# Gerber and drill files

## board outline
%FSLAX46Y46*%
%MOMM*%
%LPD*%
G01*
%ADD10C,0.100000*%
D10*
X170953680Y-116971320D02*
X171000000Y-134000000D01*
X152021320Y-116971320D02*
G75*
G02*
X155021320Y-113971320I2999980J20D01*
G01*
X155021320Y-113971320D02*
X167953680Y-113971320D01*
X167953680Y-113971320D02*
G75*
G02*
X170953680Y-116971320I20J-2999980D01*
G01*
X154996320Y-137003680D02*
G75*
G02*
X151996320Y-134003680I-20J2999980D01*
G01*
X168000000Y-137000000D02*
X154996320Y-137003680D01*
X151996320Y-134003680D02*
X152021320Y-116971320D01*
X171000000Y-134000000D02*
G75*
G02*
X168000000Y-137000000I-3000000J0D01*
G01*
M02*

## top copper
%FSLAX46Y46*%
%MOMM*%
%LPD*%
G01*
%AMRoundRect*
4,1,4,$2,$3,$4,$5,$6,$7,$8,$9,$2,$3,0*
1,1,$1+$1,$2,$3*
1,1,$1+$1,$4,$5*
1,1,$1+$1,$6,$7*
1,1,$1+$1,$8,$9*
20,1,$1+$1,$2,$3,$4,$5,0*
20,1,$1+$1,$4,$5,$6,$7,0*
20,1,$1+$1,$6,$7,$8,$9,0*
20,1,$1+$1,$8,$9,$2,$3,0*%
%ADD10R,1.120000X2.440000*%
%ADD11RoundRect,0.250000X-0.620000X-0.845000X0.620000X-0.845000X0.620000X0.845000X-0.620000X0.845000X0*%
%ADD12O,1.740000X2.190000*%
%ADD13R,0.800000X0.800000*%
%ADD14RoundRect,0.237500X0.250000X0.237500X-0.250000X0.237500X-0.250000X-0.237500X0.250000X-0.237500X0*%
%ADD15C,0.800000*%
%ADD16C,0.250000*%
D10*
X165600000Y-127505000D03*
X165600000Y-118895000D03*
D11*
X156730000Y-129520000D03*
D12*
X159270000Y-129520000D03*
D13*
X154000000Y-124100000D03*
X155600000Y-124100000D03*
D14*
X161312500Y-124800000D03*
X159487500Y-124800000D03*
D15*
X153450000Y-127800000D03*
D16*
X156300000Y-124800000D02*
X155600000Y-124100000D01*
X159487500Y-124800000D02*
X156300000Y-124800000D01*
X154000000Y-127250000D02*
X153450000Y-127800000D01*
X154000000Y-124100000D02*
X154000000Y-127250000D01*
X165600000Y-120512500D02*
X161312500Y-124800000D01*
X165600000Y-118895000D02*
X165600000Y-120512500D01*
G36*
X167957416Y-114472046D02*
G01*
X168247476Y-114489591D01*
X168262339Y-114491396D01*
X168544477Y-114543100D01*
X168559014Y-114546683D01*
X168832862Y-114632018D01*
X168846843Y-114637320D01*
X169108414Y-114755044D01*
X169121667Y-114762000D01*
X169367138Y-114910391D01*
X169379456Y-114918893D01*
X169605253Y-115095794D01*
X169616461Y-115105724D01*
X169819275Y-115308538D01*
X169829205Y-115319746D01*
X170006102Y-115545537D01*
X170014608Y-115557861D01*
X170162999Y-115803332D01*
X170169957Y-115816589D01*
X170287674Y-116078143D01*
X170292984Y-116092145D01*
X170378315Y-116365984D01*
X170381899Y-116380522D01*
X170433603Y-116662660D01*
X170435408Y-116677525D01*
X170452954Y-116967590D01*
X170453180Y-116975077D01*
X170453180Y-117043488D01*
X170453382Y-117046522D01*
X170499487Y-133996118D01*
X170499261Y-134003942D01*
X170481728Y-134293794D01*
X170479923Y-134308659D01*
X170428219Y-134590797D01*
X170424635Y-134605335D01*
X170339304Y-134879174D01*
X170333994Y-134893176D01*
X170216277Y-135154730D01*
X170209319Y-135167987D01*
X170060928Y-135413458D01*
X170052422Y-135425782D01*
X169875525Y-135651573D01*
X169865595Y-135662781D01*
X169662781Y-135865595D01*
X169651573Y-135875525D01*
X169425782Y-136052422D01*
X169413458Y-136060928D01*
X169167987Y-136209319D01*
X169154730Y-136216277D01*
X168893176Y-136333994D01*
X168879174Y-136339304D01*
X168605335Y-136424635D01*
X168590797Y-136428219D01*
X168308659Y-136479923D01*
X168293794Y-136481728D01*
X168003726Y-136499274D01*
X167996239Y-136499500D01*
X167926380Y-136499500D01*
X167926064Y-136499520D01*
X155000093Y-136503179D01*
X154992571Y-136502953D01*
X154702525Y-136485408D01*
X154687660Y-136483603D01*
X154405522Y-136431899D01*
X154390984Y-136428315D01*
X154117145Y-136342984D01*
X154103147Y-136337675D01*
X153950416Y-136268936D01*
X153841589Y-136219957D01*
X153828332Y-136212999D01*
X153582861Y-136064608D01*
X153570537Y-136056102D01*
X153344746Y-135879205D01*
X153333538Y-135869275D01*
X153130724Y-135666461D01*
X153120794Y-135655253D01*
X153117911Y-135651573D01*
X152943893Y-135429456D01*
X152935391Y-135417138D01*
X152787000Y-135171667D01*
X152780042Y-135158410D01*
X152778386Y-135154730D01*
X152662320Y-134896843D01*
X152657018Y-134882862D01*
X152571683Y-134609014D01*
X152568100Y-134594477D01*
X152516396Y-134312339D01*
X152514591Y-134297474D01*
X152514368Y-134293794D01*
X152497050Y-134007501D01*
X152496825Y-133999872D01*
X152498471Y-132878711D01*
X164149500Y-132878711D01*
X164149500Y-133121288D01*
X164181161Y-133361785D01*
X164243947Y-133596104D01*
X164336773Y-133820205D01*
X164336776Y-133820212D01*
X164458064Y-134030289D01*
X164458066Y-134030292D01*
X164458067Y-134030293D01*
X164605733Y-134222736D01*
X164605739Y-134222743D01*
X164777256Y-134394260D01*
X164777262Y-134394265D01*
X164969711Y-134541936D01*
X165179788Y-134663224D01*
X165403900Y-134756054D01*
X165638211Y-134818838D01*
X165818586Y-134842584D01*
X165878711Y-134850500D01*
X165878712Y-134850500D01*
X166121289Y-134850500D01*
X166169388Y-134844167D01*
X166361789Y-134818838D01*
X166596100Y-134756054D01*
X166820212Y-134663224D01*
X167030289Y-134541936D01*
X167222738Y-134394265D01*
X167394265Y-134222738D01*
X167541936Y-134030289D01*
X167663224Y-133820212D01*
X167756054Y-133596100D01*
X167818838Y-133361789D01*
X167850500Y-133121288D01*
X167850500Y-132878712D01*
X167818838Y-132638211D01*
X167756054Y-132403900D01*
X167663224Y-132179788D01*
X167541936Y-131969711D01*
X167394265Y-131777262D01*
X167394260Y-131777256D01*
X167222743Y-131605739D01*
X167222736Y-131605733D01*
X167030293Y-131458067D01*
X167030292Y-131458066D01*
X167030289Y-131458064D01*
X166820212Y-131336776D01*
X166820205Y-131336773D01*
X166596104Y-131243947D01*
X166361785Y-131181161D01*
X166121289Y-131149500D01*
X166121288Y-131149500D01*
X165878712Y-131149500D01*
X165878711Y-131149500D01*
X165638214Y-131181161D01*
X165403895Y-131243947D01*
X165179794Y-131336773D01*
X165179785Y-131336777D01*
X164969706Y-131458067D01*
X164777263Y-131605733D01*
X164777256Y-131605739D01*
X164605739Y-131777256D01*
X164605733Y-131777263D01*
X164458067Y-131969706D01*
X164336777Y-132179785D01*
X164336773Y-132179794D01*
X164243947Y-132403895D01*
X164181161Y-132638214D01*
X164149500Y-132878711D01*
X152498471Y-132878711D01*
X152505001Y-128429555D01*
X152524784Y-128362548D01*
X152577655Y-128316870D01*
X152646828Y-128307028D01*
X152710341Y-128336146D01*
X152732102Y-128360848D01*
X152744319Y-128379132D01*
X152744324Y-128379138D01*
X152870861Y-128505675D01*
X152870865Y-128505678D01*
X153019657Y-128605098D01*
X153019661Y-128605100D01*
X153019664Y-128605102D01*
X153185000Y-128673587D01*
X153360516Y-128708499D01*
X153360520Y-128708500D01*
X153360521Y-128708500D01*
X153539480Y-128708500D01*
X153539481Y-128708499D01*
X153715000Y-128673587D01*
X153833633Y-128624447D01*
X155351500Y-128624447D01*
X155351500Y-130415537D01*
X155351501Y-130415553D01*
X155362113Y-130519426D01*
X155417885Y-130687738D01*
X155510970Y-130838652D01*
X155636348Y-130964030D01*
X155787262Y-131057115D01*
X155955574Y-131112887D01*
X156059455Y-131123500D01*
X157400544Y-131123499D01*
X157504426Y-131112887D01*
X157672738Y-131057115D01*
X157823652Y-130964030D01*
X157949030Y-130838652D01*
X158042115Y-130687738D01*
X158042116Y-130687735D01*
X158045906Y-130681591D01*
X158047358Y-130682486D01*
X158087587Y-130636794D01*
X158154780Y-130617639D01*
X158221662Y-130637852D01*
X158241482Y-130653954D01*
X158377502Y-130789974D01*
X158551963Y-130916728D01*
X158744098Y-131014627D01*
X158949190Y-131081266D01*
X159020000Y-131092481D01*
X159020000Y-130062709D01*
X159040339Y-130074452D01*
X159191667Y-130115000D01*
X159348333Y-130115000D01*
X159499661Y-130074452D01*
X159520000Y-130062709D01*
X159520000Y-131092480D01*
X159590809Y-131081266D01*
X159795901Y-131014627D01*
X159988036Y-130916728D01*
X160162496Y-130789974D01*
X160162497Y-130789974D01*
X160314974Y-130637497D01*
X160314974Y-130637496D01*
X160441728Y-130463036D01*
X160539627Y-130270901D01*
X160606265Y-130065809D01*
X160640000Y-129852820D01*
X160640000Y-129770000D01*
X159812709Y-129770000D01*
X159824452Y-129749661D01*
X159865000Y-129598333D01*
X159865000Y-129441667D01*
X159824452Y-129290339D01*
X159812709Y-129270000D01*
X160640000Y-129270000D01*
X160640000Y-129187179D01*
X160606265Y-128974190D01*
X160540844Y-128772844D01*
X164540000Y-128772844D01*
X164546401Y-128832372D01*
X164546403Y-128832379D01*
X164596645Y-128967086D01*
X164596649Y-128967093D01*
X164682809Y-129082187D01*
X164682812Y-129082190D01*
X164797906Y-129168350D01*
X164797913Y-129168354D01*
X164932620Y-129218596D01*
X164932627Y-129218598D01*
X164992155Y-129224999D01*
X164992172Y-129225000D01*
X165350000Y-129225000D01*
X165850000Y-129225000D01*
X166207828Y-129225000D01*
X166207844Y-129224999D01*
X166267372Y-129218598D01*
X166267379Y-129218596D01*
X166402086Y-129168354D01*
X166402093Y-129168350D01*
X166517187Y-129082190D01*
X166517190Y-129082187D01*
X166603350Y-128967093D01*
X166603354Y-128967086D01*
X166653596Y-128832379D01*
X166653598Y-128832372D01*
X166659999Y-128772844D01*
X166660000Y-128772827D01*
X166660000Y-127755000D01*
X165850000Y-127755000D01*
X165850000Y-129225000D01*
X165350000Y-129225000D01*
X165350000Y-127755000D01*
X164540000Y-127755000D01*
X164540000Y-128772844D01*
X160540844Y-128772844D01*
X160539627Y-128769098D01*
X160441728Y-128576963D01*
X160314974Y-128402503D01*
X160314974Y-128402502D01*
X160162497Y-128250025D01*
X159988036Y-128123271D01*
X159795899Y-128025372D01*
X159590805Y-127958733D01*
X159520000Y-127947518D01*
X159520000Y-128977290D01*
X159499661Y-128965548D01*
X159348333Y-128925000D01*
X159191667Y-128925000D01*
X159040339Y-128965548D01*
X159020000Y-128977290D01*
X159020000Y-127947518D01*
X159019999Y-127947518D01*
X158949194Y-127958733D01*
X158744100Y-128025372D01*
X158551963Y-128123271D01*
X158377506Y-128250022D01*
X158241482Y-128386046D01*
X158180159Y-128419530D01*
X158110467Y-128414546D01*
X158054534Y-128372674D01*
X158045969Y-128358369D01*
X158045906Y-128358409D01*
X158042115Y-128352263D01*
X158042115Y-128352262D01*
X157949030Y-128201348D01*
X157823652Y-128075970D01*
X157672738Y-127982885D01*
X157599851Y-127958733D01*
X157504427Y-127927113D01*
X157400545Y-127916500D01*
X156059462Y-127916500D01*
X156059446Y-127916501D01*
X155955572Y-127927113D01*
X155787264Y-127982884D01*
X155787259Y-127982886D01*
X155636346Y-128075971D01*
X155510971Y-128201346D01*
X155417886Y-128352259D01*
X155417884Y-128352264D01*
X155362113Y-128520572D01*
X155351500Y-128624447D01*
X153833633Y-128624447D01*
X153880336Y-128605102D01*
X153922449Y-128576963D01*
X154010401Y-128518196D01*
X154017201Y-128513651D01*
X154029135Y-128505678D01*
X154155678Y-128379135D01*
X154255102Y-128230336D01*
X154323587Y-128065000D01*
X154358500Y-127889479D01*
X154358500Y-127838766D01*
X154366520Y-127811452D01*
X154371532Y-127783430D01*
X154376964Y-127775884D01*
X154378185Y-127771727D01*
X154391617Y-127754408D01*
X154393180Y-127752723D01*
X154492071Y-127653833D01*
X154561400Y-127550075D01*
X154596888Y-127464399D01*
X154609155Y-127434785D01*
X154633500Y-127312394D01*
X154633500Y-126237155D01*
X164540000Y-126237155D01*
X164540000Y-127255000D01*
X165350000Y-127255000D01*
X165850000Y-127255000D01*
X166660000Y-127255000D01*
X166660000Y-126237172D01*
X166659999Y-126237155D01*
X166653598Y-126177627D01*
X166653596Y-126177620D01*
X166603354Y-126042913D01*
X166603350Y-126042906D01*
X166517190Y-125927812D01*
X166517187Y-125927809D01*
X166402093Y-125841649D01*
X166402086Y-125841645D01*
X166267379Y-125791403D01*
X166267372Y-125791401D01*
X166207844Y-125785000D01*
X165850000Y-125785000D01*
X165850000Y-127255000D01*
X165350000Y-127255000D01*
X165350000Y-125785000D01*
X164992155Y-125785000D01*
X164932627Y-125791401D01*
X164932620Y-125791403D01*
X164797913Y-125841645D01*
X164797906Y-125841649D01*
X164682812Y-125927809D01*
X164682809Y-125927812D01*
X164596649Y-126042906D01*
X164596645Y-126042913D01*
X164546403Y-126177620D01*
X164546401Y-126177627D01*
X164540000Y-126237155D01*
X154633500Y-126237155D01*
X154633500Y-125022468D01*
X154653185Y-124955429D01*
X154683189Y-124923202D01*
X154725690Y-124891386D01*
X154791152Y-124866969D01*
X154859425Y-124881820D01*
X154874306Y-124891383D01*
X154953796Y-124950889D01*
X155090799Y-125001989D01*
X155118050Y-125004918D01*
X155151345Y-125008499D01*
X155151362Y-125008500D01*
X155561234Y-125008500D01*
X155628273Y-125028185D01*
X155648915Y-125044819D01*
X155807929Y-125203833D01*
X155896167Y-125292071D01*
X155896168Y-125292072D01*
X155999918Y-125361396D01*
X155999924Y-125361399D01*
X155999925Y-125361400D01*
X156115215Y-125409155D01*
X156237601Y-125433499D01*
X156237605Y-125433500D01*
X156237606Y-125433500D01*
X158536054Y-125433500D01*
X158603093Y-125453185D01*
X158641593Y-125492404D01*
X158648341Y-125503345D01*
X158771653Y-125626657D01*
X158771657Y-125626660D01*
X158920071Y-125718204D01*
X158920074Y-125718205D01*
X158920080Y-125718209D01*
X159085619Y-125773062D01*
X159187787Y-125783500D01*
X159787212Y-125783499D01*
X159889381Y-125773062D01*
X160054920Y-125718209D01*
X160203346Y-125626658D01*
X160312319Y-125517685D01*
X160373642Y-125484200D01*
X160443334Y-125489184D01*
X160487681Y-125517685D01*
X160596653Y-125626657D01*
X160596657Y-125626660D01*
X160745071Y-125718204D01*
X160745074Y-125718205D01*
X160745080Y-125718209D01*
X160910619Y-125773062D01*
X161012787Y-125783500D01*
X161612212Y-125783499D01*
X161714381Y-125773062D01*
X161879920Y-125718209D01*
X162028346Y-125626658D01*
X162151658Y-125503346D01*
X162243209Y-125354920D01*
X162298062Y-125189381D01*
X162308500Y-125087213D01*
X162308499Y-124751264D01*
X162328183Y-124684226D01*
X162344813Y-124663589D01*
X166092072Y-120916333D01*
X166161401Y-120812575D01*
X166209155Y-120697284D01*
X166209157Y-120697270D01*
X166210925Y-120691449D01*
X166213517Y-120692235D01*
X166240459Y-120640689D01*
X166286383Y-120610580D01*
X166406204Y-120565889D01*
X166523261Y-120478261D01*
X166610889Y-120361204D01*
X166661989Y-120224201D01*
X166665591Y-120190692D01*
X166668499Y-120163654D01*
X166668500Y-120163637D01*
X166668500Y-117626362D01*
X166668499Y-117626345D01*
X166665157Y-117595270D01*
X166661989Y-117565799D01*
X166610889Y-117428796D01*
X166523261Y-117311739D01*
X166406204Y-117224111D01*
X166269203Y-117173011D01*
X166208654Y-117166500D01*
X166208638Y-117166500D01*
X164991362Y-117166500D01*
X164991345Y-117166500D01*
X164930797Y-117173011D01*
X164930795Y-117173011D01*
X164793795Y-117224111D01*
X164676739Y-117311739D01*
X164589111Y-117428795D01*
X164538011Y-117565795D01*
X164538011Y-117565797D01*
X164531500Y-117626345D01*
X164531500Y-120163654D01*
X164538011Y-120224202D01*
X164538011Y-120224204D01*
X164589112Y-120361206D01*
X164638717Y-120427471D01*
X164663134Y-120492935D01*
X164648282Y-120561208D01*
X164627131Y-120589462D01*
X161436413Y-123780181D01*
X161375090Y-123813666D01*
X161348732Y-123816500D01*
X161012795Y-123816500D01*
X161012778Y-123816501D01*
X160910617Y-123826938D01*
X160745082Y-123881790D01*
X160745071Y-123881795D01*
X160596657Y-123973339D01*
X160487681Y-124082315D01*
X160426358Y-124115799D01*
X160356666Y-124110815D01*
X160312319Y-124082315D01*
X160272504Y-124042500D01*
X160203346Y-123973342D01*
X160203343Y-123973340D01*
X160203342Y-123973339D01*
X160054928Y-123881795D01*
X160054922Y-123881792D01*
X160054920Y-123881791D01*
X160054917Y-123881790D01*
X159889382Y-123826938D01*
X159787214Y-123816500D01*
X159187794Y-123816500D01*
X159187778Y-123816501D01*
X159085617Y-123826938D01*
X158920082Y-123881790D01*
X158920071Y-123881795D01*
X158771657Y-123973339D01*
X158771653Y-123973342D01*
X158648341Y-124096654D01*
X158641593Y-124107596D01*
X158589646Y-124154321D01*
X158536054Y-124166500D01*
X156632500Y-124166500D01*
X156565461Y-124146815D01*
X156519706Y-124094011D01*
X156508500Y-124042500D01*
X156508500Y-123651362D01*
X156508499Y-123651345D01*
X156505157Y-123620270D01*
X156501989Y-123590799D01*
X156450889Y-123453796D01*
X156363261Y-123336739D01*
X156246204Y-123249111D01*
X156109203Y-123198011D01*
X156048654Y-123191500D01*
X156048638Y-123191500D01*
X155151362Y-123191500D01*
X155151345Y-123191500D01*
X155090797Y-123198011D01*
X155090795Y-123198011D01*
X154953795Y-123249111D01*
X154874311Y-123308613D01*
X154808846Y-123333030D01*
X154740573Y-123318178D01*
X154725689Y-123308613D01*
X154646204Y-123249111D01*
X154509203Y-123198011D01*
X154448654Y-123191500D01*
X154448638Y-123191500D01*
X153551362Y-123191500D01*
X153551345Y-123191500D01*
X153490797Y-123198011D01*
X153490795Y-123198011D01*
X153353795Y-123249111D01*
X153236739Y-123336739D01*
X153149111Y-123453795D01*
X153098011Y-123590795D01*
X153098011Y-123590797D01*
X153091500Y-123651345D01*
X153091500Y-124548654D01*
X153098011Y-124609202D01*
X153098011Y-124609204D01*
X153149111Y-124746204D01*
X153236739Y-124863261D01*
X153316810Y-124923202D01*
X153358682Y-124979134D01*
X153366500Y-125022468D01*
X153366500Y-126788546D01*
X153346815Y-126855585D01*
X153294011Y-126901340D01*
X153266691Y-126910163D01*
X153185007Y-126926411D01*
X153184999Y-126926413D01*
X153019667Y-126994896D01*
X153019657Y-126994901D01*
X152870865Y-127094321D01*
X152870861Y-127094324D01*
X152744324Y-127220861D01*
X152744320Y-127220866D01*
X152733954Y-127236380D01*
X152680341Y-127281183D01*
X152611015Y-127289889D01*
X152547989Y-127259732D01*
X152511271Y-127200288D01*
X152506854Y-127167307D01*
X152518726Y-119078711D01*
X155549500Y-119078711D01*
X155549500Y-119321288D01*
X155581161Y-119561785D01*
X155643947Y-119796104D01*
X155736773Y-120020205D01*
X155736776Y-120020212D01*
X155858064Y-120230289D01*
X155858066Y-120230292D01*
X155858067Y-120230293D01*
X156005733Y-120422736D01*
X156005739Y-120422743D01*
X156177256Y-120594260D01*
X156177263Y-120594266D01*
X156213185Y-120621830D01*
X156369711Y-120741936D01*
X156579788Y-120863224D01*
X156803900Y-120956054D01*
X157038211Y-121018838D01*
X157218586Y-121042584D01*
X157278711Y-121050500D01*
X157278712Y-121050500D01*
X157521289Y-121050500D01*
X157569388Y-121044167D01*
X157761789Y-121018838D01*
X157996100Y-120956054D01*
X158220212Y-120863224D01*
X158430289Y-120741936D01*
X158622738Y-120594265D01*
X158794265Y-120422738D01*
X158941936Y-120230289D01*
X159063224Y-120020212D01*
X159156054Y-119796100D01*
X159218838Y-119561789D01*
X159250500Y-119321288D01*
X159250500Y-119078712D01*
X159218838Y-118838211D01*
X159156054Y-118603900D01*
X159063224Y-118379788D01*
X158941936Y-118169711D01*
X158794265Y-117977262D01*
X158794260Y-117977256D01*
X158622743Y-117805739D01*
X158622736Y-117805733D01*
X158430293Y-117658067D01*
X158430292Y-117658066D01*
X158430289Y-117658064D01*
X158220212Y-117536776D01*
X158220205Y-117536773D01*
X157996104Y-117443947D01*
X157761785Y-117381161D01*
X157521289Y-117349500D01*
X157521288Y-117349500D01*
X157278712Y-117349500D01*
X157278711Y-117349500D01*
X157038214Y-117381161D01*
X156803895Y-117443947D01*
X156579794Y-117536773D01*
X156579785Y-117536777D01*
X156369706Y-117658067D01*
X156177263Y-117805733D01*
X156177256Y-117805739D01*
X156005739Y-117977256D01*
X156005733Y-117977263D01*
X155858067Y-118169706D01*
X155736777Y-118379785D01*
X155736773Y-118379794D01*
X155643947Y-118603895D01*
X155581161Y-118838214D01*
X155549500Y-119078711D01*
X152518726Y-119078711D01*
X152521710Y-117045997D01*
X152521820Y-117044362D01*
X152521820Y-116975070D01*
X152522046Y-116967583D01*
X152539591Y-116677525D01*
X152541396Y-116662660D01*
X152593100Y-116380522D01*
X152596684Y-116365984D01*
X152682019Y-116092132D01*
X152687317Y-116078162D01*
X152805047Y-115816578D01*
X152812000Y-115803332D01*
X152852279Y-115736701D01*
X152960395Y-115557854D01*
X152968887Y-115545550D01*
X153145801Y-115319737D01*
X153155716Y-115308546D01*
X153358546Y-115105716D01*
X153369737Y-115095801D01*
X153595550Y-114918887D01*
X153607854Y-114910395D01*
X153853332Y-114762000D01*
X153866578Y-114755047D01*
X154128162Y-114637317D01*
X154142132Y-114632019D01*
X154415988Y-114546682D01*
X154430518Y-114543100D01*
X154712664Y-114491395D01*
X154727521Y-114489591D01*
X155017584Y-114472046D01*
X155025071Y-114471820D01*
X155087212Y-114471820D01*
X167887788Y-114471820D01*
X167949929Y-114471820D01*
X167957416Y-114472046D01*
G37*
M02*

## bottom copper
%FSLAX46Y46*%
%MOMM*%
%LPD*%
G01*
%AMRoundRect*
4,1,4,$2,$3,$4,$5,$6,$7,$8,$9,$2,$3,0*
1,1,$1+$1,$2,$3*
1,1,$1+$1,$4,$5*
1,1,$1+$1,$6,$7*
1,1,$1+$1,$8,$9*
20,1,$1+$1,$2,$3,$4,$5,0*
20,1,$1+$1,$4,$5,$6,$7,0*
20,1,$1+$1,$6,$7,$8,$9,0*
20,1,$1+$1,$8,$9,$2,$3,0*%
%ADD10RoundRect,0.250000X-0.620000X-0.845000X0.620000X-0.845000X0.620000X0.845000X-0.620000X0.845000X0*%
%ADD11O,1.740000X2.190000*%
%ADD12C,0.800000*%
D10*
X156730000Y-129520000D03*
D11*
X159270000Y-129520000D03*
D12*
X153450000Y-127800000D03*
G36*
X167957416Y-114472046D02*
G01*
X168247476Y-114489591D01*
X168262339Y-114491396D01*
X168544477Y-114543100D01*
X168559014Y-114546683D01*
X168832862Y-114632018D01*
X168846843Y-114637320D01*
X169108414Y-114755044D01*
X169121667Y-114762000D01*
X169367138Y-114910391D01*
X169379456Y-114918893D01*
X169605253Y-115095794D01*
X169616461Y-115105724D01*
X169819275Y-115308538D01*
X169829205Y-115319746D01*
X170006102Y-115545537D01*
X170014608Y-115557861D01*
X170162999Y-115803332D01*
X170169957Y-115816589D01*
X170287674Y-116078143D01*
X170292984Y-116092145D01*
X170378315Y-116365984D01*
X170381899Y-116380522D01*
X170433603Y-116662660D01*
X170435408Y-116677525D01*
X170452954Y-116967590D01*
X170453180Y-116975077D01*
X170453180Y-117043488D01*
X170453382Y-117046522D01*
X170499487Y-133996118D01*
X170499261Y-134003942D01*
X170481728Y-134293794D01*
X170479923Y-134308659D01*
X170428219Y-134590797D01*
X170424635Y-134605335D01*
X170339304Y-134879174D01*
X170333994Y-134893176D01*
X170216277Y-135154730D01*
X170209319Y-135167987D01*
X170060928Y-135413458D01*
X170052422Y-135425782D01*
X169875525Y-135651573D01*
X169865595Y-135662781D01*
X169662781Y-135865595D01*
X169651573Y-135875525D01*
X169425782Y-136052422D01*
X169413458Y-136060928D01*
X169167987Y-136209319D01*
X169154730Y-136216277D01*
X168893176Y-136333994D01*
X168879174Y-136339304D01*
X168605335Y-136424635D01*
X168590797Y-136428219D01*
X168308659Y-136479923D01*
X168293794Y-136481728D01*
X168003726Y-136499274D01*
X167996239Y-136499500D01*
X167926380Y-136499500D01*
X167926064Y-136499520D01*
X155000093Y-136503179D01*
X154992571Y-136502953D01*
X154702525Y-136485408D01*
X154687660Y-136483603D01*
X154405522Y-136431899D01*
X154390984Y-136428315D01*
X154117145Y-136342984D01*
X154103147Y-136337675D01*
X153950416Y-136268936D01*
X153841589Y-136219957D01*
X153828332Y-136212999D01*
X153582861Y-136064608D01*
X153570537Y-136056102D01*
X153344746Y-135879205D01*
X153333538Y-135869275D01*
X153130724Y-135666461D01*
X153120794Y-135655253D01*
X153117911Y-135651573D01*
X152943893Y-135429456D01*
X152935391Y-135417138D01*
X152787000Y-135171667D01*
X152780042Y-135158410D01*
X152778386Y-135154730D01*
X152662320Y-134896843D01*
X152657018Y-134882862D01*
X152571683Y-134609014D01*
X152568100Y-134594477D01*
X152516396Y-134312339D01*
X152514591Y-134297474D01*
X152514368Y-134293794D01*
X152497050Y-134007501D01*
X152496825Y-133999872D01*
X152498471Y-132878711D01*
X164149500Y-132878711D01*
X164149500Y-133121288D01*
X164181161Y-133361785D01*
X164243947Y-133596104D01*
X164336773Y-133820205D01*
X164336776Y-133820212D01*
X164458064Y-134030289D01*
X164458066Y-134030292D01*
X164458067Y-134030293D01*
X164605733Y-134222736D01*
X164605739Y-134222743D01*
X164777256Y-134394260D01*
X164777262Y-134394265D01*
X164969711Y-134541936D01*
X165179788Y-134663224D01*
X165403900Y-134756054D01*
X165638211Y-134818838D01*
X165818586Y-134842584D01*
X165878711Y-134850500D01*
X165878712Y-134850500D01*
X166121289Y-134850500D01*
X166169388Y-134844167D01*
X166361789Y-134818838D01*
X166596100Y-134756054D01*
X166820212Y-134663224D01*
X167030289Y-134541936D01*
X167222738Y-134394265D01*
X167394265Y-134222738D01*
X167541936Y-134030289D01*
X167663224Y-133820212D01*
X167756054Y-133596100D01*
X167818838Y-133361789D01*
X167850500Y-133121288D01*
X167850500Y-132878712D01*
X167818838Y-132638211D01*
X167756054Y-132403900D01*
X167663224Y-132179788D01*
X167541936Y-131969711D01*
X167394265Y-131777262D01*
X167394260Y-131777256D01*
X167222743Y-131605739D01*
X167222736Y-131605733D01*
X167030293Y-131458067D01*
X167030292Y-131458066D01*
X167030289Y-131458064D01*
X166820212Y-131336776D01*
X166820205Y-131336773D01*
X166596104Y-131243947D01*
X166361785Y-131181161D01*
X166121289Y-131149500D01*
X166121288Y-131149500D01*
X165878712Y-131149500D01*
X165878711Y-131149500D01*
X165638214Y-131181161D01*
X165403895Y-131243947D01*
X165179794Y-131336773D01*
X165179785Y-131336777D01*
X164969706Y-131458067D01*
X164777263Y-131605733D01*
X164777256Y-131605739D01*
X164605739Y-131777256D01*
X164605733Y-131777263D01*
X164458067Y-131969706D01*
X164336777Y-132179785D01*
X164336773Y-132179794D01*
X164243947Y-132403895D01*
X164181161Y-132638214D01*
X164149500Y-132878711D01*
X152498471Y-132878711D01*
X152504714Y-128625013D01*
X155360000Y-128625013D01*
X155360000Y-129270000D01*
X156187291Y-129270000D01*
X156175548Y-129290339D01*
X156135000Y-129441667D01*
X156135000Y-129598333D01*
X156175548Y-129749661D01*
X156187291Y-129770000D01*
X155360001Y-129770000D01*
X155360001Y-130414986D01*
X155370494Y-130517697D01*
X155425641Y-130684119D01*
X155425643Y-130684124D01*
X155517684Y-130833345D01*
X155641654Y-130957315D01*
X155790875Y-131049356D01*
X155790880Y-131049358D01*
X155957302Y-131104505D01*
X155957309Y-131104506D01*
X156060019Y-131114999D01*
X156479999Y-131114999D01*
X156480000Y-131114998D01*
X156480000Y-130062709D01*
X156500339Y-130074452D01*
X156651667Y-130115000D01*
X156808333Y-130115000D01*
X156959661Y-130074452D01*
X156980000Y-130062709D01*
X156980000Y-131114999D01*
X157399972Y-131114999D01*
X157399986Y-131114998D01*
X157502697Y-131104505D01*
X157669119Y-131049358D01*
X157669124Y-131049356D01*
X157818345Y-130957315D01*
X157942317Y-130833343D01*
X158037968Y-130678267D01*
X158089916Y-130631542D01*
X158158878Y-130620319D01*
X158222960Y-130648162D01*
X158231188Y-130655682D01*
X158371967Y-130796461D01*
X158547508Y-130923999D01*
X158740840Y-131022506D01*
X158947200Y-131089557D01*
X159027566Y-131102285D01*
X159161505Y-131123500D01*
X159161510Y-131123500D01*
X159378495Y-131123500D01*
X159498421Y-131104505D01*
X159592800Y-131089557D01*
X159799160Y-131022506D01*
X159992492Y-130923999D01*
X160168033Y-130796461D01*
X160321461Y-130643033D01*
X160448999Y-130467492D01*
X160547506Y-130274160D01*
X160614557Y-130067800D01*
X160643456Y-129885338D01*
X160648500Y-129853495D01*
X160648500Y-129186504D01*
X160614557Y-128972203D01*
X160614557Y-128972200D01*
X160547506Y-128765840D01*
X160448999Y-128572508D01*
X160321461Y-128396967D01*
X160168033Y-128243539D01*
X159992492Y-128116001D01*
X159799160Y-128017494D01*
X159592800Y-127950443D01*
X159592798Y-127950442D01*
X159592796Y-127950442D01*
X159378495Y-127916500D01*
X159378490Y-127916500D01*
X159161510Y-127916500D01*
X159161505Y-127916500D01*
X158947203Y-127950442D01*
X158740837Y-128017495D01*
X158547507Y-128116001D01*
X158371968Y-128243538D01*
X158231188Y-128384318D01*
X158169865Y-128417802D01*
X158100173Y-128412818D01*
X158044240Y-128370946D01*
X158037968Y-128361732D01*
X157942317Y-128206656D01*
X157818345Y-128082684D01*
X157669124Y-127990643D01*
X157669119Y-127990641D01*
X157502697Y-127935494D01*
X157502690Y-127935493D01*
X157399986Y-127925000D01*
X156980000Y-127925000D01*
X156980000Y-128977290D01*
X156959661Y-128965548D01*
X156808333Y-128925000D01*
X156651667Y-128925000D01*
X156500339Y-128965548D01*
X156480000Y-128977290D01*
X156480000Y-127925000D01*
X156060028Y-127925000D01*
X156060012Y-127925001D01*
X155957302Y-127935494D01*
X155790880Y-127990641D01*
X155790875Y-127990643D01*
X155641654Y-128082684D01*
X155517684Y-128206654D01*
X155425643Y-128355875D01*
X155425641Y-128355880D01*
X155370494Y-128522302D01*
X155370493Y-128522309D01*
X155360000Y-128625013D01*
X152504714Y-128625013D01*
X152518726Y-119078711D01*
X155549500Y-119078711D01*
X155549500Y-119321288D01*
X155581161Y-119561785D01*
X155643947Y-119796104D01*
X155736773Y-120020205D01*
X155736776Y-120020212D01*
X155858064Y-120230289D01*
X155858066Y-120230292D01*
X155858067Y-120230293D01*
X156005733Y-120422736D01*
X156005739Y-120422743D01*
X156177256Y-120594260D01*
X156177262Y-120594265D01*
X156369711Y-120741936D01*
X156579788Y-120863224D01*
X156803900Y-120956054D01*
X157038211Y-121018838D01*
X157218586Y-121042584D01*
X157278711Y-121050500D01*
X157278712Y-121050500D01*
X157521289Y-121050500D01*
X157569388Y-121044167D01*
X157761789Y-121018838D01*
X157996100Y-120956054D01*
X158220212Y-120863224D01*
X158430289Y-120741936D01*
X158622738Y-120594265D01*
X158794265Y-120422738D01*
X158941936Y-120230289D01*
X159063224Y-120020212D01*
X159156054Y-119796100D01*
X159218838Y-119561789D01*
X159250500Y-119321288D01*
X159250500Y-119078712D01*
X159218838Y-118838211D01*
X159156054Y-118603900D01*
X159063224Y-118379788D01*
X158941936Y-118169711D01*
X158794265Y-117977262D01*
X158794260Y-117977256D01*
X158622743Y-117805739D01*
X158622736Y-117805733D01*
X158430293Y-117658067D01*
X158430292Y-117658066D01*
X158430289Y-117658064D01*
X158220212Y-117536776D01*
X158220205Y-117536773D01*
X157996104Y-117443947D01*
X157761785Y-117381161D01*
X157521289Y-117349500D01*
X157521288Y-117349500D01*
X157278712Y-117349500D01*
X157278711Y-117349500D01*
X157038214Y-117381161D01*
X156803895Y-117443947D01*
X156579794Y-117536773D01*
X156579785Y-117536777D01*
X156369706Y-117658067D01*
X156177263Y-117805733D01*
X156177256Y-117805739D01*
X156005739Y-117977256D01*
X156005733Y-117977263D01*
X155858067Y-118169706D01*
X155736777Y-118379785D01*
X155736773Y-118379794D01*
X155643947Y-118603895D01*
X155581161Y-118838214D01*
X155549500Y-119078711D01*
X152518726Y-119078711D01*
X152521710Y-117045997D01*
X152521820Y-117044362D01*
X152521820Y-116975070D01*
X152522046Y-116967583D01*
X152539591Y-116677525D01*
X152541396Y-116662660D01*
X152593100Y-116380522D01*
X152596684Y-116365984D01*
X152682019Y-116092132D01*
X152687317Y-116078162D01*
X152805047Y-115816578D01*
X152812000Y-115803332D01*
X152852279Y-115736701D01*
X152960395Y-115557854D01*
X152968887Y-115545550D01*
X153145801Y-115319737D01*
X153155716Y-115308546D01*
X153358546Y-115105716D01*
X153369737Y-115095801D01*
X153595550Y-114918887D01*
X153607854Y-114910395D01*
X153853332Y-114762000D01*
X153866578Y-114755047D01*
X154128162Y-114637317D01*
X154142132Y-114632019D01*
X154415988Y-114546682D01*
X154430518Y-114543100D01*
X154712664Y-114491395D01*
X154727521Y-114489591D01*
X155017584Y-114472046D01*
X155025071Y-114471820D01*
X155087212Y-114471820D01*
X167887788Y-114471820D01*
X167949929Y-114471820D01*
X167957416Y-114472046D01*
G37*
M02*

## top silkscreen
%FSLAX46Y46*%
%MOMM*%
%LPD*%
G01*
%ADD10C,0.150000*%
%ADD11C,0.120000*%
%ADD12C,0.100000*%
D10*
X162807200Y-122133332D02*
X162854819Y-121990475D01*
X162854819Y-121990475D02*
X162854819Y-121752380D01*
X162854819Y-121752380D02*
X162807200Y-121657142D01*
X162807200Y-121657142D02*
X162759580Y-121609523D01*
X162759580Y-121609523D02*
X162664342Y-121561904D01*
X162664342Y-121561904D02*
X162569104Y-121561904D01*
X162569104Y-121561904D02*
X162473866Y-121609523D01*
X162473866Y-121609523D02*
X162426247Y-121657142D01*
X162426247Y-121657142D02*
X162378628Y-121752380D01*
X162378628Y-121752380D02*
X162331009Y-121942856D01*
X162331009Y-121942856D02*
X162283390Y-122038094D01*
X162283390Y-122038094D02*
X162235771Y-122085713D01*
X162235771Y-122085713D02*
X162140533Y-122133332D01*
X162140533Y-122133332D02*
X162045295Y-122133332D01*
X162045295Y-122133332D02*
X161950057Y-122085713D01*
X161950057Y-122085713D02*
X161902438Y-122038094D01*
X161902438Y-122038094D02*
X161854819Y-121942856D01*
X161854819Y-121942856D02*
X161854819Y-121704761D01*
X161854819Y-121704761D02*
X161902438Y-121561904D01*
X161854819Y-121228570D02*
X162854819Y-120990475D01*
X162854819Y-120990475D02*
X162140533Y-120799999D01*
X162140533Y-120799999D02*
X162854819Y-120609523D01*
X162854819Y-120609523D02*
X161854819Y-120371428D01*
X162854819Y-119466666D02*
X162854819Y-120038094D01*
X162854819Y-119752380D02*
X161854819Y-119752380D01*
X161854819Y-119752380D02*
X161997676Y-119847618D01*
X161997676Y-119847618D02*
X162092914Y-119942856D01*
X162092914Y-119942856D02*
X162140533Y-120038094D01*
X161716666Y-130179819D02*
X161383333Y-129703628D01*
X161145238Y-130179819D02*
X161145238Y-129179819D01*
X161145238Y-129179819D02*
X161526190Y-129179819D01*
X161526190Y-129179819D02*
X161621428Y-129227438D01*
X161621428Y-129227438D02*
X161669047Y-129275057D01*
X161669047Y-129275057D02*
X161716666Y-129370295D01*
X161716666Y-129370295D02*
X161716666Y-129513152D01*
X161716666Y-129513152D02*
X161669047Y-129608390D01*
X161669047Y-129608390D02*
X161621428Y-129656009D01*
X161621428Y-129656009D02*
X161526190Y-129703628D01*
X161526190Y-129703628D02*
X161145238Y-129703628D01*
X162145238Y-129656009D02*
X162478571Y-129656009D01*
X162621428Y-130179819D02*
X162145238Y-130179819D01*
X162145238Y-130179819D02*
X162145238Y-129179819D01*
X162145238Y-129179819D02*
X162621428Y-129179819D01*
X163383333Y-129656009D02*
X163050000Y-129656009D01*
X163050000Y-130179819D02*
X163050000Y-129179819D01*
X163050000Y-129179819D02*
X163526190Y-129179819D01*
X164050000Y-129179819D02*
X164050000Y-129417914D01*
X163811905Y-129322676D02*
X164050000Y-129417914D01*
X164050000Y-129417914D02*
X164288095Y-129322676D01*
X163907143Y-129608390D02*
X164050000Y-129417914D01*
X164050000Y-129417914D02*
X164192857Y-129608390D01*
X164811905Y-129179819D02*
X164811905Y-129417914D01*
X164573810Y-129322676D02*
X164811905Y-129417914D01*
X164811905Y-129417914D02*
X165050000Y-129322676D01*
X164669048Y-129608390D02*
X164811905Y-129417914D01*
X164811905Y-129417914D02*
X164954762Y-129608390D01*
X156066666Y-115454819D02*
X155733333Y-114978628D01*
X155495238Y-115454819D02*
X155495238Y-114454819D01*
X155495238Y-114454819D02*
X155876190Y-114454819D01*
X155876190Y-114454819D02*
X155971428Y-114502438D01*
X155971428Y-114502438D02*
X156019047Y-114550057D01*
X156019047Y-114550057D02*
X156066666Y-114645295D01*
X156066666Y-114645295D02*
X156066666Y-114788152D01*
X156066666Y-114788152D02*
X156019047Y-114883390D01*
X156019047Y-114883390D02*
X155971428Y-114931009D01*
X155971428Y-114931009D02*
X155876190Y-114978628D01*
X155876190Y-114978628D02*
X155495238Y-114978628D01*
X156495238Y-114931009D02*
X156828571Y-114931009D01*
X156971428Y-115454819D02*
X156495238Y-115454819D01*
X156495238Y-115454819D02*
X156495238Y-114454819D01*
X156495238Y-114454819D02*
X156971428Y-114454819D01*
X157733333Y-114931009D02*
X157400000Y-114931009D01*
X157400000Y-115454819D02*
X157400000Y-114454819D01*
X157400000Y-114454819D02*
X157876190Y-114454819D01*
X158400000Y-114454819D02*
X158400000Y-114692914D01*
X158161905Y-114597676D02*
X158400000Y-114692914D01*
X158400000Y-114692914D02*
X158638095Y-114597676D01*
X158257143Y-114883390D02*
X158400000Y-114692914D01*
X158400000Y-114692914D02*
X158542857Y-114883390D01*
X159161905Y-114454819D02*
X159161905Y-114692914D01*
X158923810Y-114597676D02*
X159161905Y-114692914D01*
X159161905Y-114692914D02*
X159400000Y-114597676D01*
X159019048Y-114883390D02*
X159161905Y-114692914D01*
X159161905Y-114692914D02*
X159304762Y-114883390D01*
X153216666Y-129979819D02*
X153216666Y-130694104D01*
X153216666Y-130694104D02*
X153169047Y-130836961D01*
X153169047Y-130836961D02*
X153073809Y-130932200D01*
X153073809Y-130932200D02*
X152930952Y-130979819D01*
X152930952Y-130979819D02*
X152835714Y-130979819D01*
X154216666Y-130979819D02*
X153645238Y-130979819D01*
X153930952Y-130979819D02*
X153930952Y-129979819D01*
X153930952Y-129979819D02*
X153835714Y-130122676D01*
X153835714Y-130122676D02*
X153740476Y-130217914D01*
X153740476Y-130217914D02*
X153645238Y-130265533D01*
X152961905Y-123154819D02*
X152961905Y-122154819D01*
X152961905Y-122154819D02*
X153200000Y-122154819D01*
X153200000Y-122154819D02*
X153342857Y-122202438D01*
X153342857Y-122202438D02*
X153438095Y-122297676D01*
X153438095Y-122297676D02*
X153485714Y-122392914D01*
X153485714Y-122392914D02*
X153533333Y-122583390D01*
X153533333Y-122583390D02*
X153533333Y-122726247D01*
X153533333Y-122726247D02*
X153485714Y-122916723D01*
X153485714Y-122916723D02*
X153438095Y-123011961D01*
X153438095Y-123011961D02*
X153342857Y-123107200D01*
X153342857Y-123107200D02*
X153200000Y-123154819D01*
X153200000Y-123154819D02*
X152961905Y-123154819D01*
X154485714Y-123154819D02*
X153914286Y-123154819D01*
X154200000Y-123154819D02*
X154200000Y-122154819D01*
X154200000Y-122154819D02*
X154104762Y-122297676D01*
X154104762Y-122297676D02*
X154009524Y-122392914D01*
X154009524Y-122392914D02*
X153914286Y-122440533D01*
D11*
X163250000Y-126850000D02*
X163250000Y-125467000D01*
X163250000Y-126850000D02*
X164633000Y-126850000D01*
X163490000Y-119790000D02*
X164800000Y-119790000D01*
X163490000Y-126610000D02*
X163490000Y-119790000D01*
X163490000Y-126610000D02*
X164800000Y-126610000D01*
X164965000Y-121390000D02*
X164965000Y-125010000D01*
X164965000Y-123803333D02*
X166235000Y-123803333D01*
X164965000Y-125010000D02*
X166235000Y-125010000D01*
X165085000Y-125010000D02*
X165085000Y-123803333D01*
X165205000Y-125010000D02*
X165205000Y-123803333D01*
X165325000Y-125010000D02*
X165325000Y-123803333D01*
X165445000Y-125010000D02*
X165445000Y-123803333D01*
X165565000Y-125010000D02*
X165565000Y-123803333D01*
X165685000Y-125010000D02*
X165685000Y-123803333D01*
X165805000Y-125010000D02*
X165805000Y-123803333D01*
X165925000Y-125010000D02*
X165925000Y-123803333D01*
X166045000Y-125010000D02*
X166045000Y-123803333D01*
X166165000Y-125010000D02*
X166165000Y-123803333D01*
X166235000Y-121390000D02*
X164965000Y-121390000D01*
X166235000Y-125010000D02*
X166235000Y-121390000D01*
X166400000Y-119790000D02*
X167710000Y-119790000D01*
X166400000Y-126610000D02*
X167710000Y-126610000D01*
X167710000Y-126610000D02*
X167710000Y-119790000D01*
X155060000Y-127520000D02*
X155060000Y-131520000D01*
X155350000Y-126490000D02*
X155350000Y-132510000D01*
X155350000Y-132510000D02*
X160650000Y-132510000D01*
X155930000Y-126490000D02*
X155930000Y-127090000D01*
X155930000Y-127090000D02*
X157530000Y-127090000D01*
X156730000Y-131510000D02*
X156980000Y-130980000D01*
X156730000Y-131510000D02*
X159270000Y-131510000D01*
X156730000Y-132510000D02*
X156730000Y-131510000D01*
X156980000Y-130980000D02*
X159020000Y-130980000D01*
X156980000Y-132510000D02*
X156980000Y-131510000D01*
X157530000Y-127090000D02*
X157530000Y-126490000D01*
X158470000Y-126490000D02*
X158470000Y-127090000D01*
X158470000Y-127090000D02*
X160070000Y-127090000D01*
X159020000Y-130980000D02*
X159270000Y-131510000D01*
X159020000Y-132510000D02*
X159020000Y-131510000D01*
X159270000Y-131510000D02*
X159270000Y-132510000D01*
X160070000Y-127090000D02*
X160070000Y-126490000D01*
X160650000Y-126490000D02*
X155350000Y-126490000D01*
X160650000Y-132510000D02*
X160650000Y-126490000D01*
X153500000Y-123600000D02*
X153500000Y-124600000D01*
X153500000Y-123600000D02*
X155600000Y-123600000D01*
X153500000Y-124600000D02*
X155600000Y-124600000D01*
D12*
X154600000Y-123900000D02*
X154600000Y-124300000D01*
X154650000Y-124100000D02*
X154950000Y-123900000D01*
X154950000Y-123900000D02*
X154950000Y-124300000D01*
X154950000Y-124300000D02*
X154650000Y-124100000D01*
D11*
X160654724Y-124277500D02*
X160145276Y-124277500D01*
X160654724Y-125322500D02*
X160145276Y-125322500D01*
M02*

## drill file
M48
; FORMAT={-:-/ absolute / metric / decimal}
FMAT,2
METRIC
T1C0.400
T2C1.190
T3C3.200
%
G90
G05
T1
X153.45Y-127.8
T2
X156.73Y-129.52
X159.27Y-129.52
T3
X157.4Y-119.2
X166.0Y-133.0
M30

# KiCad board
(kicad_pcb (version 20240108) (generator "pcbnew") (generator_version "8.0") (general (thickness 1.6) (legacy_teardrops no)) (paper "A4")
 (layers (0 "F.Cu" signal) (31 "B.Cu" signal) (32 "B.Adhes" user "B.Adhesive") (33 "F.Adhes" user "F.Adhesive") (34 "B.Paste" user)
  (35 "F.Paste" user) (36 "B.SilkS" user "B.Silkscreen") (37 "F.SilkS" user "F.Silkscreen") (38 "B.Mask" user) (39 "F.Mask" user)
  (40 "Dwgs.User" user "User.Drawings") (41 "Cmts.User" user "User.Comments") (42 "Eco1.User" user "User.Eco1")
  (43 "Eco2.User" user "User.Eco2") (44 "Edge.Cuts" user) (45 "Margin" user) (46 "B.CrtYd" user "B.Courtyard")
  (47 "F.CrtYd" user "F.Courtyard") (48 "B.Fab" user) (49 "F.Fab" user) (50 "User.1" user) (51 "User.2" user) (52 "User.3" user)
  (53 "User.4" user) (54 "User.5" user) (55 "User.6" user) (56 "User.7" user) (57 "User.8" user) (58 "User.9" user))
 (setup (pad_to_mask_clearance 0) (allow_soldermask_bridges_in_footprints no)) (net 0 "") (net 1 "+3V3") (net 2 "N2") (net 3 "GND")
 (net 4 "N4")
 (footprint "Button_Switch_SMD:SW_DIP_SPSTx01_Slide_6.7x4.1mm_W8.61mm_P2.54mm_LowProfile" (layer "F.Cu") (at 165.6 123.2 90)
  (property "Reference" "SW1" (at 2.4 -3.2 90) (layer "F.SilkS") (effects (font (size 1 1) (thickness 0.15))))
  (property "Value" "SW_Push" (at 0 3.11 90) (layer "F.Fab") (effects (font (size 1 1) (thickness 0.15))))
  (fp_line (start -3.65 -2.35) (end -2.267 -2.35) (stroke (width 0.12) (type solid)) (layer "F.SilkS"))
  (fp_line (start -3.65 -2.35) (end -3.65 -0.967) (stroke (width 0.12) (type solid)) (layer "F.SilkS"))
  (fp_line (start 3.41 -2.11) (end 3.41 -0.8) (stroke (width 0.12) (type solid)) (layer "F.SilkS"))
  (fp_line (start -3.41 -2.11) (end 3.41 -2.11) (stroke (width 0.12) (type solid)) (layer "F.SilkS"))
  (fp_line (start -3.41 -2.11) (end -3.41 -0.8) (stroke (width 0.12) (type solid)) (layer "F.SilkS"))
  (fp_line (start 1.81 -0.635) (end -1.81 -0.635) (stroke (width 0.12) (type solid)) (layer "F.SilkS"))
  (fp_line (start -0.603333 -0.635) (end -0.603333 0.635) (stroke (width 0.12) (type solid)) (layer "F.SilkS"))
  (fp_line (start -1.81 -0.635) (end -1.81 0.635) (stroke (width 0.12) (type solid)) (layer "F.SilkS"))
  (fp_line (start -1.81 -0.515) (end -0.603333 -0.515) (stroke (width 0.12) (type solid)) (layer "F.SilkS"))
  (fp_line (start -1.81 -0.395) (end -0.603333 -0.395) (stroke (width 0.12) (type solid)) (layer "F.SilkS"))
  (fp_line (start -1.81 -0.275) (end -0.603333 -0.275) (stroke (width 0.12) (type solid)) (layer "F.SilkS"))
  (fp_line (start -1.81 -0.155) (end -0.603333 -0.155) (stroke (width 0.12) (type solid)) (layer "F.SilkS"))
  (fp_line (start -1.81 -0.035) (end -0.603333 -0.035) (stroke (width 0.12) (type solid)) (layer "F.SilkS"))
  (fp_line (start -1.81 0.085) (end -0.603333 0.085) (stroke (width 0.12) (type solid)) (layer "F.SilkS"))
  (fp_line (start -1.81 0.205) (end -0.603333 0.205) (stroke (width 0.12) (type solid)) (layer "F.SilkS"))
  (fp_line (start -1.81 0.325) (end -0.603333 0.325) (stroke (width 0.12) (type solid)) (layer "F.SilkS"))
  (fp_line (start -1.81 0.445) (end -0.603333 0.445) (stroke (width 0.12) (type solid)) (layer "F.SilkS"))
  (fp_line (start -1.81 0.565) (end -0.603333 0.565) (stroke (width 0.12) (type solid)) (layer "F.SilkS"))
  (fp_line (start 1.81 0.635) (end 1.81 -0.635) (stroke (width 0.12) (type solid)) (layer "F.SilkS"))
  (fp_line (start -1.81 0.635) (end 1.81 0.635) (stroke (width 0.12) (type solid)) (layer "F.SilkS"))
  (fp_line (start 3.41 0.8) (end 3.41 2.11) (stroke (width 0.12) (type solid)) (layer "F.SilkS"))
  (fp_line (start -3.41 0.8) (end -3.41 2.11) (stroke (width 0.12) (type solid)) (layer "F.SilkS"))
  (fp_line (start -3.41 2.11) (end 3.41 2.11) (stroke (width 0.12) (type solid)) (layer "F.SilkS"))
  (pad "1" smd rect (at -4.305 0 90) (size 2.44 1.12) (layers "F.Cu" "F.Paste" "F.Mask") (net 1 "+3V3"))
  (pad "2" smd rect (at 4.305 0 90) (size 2.44 1.12) (layers "F.Cu" "F.Paste" "F.Mask") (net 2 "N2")))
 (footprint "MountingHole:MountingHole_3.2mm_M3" (layer "F.Cu") (at 166 133)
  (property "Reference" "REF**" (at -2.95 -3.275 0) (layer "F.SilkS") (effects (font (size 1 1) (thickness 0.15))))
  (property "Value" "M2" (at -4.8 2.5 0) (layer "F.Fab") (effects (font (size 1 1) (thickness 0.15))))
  (pad "" np_thru_hole circle (at 0 0) (size 3.2 3.2) (drill 3.2) (layers "*.Cu" "*.Mask")))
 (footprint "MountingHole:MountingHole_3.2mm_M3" (layer "F.Cu") (at 157.4 119.2)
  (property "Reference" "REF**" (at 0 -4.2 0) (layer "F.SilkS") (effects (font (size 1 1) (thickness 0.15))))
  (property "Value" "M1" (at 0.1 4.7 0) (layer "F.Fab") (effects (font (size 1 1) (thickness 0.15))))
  (pad "" np_thru_hole circle (at 0 0) (size 3.2 3.2) (drill 3.2) (layers "*.Cu" "*.Mask")))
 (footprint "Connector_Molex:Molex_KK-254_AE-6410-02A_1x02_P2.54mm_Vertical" (layer "F.Cu") (at 156.73 129.52)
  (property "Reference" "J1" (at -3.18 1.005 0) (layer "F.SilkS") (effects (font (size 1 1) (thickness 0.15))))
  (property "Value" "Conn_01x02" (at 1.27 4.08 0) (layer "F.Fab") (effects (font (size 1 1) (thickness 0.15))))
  (fp_line (start -1.67 -2) (end -1.67 2) (stroke (width 0.12) (type solid)) (layer "F.SilkS"))
  (fp_line (start -1.38 -3.03) (end -1.38 2.99) (stroke (width 0.12) (type solid)) (layer "F.SilkS"))
  (fp_line (start -1.38 2.99) (end 3.92 2.99) (stroke (width 0.12) (type solid)) (layer "F.SilkS"))
  (fp_line (start -0.8 -3.03) (end -0.8 -2.43) (stroke (width 0.12) (type solid)) (layer "F.SilkS"))
  (fp_line (start -0.8 -2.43) (end 0.8 -2.43) (stroke (width 0.12) (type solid)) (layer "F.SilkS"))
  (fp_line (start 0 1.99) (end 0.25 1.46) (stroke (width 0.12) (type solid)) (layer "F.SilkS"))
  (fp_line (start 0 1.99) (end 2.54 1.99) (stroke (width 0.12) (type solid)) (layer "F.SilkS"))
  (fp_line (start 0 2.99) (end 0 1.99) (stroke (width 0.12) (type solid)) (layer "F.SilkS"))
  (fp_line (start 0.25 1.46) (end 2.29 1.46) (stroke (width 0.12) (type solid)) (layer "F.SilkS"))
  (fp_line (start 0.25 2.99) (end 0.25 1.99) (stroke (width 0.12) (type solid)) (layer "F.SilkS"))
  (fp_line (start 0.8 -2.43) (end 0.8 -3.03) (stroke (width 0.12) (type solid)) (layer "F.SilkS"))
  (fp_line (start 1.74 -3.03) (end 1.74 -2.43) (stroke (width 0.12) (type solid)) (layer "F.SilkS"))
  (fp_line (start 1.74 -2.43) (end 3.34 -2.43) (stroke (width 0.12) (type solid)) (layer "F.SilkS"))
  (fp_line (start 2.29 1.46) (end 2.54 1.99) (stroke (width 0.12) (type solid)) (layer "F.SilkS"))
  (fp_line (start 2.29 2.99) (end 2.29 1.99) (stroke (width 0.12) (type solid)) (layer "F.SilkS"))
  (fp_line (start 2.54 1.99) (end 2.54 2.99) (stroke (width 0.12) (type solid)) (layer "F.SilkS"))
  (fp_line (start 3.34 -2.43) (end 3.34 -3.03) (stroke (width 0.12) (type solid)) (layer "F.SilkS"))
  (fp_line (start 3.92 -3.03) (end -1.38 -3.03) (stroke (width 0.12) (type solid)) (layer "F.SilkS"))
  (fp_line (start 3.92 2.99) (end 3.92 -3.03) (stroke (width 0.12) (type solid)) (layer "F.SilkS"))
  (pad "1" thru_hole roundrect (at 0 0) (size 1.74 2.19) (drill 1.19) (layers "*.Cu" "*.Mask") (remove_unused_layers no)
   (roundrect_rratio 0.143678) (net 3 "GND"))
  (pad "2" thru_hole oval (at 2.54 0) (size 1.74 2.19) (drill 1.19) (layers "*.Cu" "*.Mask") (remove_unused_layers no) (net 1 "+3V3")))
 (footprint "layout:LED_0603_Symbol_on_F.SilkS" (layer "F.Cu") (at 154.8 124.1)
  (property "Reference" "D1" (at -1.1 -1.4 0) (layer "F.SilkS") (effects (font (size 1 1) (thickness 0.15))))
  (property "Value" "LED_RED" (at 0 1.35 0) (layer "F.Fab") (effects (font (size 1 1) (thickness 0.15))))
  (fp_line (start -1.3 -0.5) (end -1.3 0.5) (stroke (width 0.12) (type solid)) (layer "F.SilkS"))
  (fp_line (start -1.3 -0.5) (end 0.8 -0.5) (stroke (width 0.12) (type solid)) (layer "F.SilkS"))
  (fp_line (start -1.3 0.5) (end 0.8 0.5) (stroke (width 0.12) (type solid)) (layer "F.SilkS"))
  (fp_line (start -0.2 -0.2) (end -0.2 0.2) (stroke (width 0.1) (type solid)) (layer "F.SilkS"))
  (fp_line (start -0.15 0) (end 0.15 -0.2) (stroke (width 0.1) (type solid)) (layer "F.SilkS"))
  (fp_line (start 0.15 -0.2) (end 0.15 0.2) (stroke (width 0.1) (type solid)) (layer "F.SilkS"))
  (fp_line (start 0.15 0.2) (end -0.15 0) (stroke (width 0.1) (type solid)) (layer "F.SilkS"))
  (pad "1" smd rect (at -0.8 0 180) (size 0.8 0.8) (layers "F.Cu" "F.Paste" "F.Mask") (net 3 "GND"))
  (pad "2" smd rect (at 0.8 0 180) (size 0.8 0.8) (layers "F.Cu" "F.Paste" "F.Mask") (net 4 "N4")))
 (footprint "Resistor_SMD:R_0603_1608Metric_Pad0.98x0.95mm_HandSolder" (layer "F.Cu") (at 160.4 124.8 180)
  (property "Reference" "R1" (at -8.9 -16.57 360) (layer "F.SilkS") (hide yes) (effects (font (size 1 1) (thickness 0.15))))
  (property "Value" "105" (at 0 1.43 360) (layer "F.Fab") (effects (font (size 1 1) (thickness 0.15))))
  (fp_line (start -0.254724 0.5225) (end 0.254724 0.5225) (stroke (width 0.12) (type solid)) (layer "F.SilkS"))
  (fp_line (start -0.254724 -0.5225) (end 0.254724 -0.5225) (stroke (width 0.12) (type solid)) (layer "F.SilkS"))
  (pad "1" smd roundrect (at -0.9125 0 180) (size 0.975 0.95) (layers "F.Cu" "F.Paste" "F.Mask") (roundrect_rratio 0.25) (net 2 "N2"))
  (pad "2" smd roundrect (at 0.9125 0 180) (size 0.975 0.95) (layers "F.Cu" "F.Paste" "F.Mask") (roundrect_rratio 0.25) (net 4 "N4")))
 (gr_line (start 170.95368 116.97132) (end 171 134) (stroke (width 0.1) (type default)) (layer "Edge.Cuts"))
 (gr_arc (start 152.02132 116.97132) (mid 152.9 114.85) (end 155.02132 113.97132) (stroke (width 0.1) (type default)) (layer "Edge.Cuts"))
 (gr_line (start 155.02132 113.97132) (end 167.95368 113.97132) (stroke (width 0.1) (type default)) (layer "Edge.Cuts"))
 (gr_arc (start 167.95368 113.97132) (mid 170.075 114.85) (end 170.95368 116.97132) (stroke (width 0.1) (type default)) (layer "Edge.Cuts"))
 (gr_arc (start 154.99632 137.00368) (mid 152.875 136.125) (end 151.99632 134.00368) (stroke (width 0.1) (type default)) (layer "Edge.Cuts"))
 (gr_line (start 168 137) (end 154.99632 137.00368) (stroke (width 0.1) (type default)) (layer "Edge.Cuts"))
 (gr_line (start 151.99632 134.00368) (end 152.02132 116.97132) (stroke (width 0.1) (type default)) (layer "Edge.Cuts"))
 (gr_arc (start 171 134) (mid 170.12132 136.12132) (end 168 137) (stroke (width 0.1) (type default)) (layer "Edge.Cuts"))
 (segment (start 156.3 124.8) (end 155.6 124.1) (width 0.25) (layer "F.Cu") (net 4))
 (segment (start 159.4875 124.8) (end 156.3 124.8) (width 0.25) (layer "F.Cu") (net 4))
 (segment (start 154 127.25) (end 153.45 127.8) (width 0.25) (layer "F.Cu") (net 3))
 (segment (start 154 124.1) (end 154 127.25) (width 0.25) (layer "F.Cu") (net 3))
 (via (at 153.45 127.8) (size 0.8) (drill 0.4) (layers "F.Cu" "B.Cu") (free yes) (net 3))
 (segment (start 165.6 120.5125) (end 161.3125 124.8) (width 0.25) (layer "F.Cu") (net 2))
 (segment (start 165.6 118.895) (end 165.6 120.5125) (width 0.25) (layer "F.Cu") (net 2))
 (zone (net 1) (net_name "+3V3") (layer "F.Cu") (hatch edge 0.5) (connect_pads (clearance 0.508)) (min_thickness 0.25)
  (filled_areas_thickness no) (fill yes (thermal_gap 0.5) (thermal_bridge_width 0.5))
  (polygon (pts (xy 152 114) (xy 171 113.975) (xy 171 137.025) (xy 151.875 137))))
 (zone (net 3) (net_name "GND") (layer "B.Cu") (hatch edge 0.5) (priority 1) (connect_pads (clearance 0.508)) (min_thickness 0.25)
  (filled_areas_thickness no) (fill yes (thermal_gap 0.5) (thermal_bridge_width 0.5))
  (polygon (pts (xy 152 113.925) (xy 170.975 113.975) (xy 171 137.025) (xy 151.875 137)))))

